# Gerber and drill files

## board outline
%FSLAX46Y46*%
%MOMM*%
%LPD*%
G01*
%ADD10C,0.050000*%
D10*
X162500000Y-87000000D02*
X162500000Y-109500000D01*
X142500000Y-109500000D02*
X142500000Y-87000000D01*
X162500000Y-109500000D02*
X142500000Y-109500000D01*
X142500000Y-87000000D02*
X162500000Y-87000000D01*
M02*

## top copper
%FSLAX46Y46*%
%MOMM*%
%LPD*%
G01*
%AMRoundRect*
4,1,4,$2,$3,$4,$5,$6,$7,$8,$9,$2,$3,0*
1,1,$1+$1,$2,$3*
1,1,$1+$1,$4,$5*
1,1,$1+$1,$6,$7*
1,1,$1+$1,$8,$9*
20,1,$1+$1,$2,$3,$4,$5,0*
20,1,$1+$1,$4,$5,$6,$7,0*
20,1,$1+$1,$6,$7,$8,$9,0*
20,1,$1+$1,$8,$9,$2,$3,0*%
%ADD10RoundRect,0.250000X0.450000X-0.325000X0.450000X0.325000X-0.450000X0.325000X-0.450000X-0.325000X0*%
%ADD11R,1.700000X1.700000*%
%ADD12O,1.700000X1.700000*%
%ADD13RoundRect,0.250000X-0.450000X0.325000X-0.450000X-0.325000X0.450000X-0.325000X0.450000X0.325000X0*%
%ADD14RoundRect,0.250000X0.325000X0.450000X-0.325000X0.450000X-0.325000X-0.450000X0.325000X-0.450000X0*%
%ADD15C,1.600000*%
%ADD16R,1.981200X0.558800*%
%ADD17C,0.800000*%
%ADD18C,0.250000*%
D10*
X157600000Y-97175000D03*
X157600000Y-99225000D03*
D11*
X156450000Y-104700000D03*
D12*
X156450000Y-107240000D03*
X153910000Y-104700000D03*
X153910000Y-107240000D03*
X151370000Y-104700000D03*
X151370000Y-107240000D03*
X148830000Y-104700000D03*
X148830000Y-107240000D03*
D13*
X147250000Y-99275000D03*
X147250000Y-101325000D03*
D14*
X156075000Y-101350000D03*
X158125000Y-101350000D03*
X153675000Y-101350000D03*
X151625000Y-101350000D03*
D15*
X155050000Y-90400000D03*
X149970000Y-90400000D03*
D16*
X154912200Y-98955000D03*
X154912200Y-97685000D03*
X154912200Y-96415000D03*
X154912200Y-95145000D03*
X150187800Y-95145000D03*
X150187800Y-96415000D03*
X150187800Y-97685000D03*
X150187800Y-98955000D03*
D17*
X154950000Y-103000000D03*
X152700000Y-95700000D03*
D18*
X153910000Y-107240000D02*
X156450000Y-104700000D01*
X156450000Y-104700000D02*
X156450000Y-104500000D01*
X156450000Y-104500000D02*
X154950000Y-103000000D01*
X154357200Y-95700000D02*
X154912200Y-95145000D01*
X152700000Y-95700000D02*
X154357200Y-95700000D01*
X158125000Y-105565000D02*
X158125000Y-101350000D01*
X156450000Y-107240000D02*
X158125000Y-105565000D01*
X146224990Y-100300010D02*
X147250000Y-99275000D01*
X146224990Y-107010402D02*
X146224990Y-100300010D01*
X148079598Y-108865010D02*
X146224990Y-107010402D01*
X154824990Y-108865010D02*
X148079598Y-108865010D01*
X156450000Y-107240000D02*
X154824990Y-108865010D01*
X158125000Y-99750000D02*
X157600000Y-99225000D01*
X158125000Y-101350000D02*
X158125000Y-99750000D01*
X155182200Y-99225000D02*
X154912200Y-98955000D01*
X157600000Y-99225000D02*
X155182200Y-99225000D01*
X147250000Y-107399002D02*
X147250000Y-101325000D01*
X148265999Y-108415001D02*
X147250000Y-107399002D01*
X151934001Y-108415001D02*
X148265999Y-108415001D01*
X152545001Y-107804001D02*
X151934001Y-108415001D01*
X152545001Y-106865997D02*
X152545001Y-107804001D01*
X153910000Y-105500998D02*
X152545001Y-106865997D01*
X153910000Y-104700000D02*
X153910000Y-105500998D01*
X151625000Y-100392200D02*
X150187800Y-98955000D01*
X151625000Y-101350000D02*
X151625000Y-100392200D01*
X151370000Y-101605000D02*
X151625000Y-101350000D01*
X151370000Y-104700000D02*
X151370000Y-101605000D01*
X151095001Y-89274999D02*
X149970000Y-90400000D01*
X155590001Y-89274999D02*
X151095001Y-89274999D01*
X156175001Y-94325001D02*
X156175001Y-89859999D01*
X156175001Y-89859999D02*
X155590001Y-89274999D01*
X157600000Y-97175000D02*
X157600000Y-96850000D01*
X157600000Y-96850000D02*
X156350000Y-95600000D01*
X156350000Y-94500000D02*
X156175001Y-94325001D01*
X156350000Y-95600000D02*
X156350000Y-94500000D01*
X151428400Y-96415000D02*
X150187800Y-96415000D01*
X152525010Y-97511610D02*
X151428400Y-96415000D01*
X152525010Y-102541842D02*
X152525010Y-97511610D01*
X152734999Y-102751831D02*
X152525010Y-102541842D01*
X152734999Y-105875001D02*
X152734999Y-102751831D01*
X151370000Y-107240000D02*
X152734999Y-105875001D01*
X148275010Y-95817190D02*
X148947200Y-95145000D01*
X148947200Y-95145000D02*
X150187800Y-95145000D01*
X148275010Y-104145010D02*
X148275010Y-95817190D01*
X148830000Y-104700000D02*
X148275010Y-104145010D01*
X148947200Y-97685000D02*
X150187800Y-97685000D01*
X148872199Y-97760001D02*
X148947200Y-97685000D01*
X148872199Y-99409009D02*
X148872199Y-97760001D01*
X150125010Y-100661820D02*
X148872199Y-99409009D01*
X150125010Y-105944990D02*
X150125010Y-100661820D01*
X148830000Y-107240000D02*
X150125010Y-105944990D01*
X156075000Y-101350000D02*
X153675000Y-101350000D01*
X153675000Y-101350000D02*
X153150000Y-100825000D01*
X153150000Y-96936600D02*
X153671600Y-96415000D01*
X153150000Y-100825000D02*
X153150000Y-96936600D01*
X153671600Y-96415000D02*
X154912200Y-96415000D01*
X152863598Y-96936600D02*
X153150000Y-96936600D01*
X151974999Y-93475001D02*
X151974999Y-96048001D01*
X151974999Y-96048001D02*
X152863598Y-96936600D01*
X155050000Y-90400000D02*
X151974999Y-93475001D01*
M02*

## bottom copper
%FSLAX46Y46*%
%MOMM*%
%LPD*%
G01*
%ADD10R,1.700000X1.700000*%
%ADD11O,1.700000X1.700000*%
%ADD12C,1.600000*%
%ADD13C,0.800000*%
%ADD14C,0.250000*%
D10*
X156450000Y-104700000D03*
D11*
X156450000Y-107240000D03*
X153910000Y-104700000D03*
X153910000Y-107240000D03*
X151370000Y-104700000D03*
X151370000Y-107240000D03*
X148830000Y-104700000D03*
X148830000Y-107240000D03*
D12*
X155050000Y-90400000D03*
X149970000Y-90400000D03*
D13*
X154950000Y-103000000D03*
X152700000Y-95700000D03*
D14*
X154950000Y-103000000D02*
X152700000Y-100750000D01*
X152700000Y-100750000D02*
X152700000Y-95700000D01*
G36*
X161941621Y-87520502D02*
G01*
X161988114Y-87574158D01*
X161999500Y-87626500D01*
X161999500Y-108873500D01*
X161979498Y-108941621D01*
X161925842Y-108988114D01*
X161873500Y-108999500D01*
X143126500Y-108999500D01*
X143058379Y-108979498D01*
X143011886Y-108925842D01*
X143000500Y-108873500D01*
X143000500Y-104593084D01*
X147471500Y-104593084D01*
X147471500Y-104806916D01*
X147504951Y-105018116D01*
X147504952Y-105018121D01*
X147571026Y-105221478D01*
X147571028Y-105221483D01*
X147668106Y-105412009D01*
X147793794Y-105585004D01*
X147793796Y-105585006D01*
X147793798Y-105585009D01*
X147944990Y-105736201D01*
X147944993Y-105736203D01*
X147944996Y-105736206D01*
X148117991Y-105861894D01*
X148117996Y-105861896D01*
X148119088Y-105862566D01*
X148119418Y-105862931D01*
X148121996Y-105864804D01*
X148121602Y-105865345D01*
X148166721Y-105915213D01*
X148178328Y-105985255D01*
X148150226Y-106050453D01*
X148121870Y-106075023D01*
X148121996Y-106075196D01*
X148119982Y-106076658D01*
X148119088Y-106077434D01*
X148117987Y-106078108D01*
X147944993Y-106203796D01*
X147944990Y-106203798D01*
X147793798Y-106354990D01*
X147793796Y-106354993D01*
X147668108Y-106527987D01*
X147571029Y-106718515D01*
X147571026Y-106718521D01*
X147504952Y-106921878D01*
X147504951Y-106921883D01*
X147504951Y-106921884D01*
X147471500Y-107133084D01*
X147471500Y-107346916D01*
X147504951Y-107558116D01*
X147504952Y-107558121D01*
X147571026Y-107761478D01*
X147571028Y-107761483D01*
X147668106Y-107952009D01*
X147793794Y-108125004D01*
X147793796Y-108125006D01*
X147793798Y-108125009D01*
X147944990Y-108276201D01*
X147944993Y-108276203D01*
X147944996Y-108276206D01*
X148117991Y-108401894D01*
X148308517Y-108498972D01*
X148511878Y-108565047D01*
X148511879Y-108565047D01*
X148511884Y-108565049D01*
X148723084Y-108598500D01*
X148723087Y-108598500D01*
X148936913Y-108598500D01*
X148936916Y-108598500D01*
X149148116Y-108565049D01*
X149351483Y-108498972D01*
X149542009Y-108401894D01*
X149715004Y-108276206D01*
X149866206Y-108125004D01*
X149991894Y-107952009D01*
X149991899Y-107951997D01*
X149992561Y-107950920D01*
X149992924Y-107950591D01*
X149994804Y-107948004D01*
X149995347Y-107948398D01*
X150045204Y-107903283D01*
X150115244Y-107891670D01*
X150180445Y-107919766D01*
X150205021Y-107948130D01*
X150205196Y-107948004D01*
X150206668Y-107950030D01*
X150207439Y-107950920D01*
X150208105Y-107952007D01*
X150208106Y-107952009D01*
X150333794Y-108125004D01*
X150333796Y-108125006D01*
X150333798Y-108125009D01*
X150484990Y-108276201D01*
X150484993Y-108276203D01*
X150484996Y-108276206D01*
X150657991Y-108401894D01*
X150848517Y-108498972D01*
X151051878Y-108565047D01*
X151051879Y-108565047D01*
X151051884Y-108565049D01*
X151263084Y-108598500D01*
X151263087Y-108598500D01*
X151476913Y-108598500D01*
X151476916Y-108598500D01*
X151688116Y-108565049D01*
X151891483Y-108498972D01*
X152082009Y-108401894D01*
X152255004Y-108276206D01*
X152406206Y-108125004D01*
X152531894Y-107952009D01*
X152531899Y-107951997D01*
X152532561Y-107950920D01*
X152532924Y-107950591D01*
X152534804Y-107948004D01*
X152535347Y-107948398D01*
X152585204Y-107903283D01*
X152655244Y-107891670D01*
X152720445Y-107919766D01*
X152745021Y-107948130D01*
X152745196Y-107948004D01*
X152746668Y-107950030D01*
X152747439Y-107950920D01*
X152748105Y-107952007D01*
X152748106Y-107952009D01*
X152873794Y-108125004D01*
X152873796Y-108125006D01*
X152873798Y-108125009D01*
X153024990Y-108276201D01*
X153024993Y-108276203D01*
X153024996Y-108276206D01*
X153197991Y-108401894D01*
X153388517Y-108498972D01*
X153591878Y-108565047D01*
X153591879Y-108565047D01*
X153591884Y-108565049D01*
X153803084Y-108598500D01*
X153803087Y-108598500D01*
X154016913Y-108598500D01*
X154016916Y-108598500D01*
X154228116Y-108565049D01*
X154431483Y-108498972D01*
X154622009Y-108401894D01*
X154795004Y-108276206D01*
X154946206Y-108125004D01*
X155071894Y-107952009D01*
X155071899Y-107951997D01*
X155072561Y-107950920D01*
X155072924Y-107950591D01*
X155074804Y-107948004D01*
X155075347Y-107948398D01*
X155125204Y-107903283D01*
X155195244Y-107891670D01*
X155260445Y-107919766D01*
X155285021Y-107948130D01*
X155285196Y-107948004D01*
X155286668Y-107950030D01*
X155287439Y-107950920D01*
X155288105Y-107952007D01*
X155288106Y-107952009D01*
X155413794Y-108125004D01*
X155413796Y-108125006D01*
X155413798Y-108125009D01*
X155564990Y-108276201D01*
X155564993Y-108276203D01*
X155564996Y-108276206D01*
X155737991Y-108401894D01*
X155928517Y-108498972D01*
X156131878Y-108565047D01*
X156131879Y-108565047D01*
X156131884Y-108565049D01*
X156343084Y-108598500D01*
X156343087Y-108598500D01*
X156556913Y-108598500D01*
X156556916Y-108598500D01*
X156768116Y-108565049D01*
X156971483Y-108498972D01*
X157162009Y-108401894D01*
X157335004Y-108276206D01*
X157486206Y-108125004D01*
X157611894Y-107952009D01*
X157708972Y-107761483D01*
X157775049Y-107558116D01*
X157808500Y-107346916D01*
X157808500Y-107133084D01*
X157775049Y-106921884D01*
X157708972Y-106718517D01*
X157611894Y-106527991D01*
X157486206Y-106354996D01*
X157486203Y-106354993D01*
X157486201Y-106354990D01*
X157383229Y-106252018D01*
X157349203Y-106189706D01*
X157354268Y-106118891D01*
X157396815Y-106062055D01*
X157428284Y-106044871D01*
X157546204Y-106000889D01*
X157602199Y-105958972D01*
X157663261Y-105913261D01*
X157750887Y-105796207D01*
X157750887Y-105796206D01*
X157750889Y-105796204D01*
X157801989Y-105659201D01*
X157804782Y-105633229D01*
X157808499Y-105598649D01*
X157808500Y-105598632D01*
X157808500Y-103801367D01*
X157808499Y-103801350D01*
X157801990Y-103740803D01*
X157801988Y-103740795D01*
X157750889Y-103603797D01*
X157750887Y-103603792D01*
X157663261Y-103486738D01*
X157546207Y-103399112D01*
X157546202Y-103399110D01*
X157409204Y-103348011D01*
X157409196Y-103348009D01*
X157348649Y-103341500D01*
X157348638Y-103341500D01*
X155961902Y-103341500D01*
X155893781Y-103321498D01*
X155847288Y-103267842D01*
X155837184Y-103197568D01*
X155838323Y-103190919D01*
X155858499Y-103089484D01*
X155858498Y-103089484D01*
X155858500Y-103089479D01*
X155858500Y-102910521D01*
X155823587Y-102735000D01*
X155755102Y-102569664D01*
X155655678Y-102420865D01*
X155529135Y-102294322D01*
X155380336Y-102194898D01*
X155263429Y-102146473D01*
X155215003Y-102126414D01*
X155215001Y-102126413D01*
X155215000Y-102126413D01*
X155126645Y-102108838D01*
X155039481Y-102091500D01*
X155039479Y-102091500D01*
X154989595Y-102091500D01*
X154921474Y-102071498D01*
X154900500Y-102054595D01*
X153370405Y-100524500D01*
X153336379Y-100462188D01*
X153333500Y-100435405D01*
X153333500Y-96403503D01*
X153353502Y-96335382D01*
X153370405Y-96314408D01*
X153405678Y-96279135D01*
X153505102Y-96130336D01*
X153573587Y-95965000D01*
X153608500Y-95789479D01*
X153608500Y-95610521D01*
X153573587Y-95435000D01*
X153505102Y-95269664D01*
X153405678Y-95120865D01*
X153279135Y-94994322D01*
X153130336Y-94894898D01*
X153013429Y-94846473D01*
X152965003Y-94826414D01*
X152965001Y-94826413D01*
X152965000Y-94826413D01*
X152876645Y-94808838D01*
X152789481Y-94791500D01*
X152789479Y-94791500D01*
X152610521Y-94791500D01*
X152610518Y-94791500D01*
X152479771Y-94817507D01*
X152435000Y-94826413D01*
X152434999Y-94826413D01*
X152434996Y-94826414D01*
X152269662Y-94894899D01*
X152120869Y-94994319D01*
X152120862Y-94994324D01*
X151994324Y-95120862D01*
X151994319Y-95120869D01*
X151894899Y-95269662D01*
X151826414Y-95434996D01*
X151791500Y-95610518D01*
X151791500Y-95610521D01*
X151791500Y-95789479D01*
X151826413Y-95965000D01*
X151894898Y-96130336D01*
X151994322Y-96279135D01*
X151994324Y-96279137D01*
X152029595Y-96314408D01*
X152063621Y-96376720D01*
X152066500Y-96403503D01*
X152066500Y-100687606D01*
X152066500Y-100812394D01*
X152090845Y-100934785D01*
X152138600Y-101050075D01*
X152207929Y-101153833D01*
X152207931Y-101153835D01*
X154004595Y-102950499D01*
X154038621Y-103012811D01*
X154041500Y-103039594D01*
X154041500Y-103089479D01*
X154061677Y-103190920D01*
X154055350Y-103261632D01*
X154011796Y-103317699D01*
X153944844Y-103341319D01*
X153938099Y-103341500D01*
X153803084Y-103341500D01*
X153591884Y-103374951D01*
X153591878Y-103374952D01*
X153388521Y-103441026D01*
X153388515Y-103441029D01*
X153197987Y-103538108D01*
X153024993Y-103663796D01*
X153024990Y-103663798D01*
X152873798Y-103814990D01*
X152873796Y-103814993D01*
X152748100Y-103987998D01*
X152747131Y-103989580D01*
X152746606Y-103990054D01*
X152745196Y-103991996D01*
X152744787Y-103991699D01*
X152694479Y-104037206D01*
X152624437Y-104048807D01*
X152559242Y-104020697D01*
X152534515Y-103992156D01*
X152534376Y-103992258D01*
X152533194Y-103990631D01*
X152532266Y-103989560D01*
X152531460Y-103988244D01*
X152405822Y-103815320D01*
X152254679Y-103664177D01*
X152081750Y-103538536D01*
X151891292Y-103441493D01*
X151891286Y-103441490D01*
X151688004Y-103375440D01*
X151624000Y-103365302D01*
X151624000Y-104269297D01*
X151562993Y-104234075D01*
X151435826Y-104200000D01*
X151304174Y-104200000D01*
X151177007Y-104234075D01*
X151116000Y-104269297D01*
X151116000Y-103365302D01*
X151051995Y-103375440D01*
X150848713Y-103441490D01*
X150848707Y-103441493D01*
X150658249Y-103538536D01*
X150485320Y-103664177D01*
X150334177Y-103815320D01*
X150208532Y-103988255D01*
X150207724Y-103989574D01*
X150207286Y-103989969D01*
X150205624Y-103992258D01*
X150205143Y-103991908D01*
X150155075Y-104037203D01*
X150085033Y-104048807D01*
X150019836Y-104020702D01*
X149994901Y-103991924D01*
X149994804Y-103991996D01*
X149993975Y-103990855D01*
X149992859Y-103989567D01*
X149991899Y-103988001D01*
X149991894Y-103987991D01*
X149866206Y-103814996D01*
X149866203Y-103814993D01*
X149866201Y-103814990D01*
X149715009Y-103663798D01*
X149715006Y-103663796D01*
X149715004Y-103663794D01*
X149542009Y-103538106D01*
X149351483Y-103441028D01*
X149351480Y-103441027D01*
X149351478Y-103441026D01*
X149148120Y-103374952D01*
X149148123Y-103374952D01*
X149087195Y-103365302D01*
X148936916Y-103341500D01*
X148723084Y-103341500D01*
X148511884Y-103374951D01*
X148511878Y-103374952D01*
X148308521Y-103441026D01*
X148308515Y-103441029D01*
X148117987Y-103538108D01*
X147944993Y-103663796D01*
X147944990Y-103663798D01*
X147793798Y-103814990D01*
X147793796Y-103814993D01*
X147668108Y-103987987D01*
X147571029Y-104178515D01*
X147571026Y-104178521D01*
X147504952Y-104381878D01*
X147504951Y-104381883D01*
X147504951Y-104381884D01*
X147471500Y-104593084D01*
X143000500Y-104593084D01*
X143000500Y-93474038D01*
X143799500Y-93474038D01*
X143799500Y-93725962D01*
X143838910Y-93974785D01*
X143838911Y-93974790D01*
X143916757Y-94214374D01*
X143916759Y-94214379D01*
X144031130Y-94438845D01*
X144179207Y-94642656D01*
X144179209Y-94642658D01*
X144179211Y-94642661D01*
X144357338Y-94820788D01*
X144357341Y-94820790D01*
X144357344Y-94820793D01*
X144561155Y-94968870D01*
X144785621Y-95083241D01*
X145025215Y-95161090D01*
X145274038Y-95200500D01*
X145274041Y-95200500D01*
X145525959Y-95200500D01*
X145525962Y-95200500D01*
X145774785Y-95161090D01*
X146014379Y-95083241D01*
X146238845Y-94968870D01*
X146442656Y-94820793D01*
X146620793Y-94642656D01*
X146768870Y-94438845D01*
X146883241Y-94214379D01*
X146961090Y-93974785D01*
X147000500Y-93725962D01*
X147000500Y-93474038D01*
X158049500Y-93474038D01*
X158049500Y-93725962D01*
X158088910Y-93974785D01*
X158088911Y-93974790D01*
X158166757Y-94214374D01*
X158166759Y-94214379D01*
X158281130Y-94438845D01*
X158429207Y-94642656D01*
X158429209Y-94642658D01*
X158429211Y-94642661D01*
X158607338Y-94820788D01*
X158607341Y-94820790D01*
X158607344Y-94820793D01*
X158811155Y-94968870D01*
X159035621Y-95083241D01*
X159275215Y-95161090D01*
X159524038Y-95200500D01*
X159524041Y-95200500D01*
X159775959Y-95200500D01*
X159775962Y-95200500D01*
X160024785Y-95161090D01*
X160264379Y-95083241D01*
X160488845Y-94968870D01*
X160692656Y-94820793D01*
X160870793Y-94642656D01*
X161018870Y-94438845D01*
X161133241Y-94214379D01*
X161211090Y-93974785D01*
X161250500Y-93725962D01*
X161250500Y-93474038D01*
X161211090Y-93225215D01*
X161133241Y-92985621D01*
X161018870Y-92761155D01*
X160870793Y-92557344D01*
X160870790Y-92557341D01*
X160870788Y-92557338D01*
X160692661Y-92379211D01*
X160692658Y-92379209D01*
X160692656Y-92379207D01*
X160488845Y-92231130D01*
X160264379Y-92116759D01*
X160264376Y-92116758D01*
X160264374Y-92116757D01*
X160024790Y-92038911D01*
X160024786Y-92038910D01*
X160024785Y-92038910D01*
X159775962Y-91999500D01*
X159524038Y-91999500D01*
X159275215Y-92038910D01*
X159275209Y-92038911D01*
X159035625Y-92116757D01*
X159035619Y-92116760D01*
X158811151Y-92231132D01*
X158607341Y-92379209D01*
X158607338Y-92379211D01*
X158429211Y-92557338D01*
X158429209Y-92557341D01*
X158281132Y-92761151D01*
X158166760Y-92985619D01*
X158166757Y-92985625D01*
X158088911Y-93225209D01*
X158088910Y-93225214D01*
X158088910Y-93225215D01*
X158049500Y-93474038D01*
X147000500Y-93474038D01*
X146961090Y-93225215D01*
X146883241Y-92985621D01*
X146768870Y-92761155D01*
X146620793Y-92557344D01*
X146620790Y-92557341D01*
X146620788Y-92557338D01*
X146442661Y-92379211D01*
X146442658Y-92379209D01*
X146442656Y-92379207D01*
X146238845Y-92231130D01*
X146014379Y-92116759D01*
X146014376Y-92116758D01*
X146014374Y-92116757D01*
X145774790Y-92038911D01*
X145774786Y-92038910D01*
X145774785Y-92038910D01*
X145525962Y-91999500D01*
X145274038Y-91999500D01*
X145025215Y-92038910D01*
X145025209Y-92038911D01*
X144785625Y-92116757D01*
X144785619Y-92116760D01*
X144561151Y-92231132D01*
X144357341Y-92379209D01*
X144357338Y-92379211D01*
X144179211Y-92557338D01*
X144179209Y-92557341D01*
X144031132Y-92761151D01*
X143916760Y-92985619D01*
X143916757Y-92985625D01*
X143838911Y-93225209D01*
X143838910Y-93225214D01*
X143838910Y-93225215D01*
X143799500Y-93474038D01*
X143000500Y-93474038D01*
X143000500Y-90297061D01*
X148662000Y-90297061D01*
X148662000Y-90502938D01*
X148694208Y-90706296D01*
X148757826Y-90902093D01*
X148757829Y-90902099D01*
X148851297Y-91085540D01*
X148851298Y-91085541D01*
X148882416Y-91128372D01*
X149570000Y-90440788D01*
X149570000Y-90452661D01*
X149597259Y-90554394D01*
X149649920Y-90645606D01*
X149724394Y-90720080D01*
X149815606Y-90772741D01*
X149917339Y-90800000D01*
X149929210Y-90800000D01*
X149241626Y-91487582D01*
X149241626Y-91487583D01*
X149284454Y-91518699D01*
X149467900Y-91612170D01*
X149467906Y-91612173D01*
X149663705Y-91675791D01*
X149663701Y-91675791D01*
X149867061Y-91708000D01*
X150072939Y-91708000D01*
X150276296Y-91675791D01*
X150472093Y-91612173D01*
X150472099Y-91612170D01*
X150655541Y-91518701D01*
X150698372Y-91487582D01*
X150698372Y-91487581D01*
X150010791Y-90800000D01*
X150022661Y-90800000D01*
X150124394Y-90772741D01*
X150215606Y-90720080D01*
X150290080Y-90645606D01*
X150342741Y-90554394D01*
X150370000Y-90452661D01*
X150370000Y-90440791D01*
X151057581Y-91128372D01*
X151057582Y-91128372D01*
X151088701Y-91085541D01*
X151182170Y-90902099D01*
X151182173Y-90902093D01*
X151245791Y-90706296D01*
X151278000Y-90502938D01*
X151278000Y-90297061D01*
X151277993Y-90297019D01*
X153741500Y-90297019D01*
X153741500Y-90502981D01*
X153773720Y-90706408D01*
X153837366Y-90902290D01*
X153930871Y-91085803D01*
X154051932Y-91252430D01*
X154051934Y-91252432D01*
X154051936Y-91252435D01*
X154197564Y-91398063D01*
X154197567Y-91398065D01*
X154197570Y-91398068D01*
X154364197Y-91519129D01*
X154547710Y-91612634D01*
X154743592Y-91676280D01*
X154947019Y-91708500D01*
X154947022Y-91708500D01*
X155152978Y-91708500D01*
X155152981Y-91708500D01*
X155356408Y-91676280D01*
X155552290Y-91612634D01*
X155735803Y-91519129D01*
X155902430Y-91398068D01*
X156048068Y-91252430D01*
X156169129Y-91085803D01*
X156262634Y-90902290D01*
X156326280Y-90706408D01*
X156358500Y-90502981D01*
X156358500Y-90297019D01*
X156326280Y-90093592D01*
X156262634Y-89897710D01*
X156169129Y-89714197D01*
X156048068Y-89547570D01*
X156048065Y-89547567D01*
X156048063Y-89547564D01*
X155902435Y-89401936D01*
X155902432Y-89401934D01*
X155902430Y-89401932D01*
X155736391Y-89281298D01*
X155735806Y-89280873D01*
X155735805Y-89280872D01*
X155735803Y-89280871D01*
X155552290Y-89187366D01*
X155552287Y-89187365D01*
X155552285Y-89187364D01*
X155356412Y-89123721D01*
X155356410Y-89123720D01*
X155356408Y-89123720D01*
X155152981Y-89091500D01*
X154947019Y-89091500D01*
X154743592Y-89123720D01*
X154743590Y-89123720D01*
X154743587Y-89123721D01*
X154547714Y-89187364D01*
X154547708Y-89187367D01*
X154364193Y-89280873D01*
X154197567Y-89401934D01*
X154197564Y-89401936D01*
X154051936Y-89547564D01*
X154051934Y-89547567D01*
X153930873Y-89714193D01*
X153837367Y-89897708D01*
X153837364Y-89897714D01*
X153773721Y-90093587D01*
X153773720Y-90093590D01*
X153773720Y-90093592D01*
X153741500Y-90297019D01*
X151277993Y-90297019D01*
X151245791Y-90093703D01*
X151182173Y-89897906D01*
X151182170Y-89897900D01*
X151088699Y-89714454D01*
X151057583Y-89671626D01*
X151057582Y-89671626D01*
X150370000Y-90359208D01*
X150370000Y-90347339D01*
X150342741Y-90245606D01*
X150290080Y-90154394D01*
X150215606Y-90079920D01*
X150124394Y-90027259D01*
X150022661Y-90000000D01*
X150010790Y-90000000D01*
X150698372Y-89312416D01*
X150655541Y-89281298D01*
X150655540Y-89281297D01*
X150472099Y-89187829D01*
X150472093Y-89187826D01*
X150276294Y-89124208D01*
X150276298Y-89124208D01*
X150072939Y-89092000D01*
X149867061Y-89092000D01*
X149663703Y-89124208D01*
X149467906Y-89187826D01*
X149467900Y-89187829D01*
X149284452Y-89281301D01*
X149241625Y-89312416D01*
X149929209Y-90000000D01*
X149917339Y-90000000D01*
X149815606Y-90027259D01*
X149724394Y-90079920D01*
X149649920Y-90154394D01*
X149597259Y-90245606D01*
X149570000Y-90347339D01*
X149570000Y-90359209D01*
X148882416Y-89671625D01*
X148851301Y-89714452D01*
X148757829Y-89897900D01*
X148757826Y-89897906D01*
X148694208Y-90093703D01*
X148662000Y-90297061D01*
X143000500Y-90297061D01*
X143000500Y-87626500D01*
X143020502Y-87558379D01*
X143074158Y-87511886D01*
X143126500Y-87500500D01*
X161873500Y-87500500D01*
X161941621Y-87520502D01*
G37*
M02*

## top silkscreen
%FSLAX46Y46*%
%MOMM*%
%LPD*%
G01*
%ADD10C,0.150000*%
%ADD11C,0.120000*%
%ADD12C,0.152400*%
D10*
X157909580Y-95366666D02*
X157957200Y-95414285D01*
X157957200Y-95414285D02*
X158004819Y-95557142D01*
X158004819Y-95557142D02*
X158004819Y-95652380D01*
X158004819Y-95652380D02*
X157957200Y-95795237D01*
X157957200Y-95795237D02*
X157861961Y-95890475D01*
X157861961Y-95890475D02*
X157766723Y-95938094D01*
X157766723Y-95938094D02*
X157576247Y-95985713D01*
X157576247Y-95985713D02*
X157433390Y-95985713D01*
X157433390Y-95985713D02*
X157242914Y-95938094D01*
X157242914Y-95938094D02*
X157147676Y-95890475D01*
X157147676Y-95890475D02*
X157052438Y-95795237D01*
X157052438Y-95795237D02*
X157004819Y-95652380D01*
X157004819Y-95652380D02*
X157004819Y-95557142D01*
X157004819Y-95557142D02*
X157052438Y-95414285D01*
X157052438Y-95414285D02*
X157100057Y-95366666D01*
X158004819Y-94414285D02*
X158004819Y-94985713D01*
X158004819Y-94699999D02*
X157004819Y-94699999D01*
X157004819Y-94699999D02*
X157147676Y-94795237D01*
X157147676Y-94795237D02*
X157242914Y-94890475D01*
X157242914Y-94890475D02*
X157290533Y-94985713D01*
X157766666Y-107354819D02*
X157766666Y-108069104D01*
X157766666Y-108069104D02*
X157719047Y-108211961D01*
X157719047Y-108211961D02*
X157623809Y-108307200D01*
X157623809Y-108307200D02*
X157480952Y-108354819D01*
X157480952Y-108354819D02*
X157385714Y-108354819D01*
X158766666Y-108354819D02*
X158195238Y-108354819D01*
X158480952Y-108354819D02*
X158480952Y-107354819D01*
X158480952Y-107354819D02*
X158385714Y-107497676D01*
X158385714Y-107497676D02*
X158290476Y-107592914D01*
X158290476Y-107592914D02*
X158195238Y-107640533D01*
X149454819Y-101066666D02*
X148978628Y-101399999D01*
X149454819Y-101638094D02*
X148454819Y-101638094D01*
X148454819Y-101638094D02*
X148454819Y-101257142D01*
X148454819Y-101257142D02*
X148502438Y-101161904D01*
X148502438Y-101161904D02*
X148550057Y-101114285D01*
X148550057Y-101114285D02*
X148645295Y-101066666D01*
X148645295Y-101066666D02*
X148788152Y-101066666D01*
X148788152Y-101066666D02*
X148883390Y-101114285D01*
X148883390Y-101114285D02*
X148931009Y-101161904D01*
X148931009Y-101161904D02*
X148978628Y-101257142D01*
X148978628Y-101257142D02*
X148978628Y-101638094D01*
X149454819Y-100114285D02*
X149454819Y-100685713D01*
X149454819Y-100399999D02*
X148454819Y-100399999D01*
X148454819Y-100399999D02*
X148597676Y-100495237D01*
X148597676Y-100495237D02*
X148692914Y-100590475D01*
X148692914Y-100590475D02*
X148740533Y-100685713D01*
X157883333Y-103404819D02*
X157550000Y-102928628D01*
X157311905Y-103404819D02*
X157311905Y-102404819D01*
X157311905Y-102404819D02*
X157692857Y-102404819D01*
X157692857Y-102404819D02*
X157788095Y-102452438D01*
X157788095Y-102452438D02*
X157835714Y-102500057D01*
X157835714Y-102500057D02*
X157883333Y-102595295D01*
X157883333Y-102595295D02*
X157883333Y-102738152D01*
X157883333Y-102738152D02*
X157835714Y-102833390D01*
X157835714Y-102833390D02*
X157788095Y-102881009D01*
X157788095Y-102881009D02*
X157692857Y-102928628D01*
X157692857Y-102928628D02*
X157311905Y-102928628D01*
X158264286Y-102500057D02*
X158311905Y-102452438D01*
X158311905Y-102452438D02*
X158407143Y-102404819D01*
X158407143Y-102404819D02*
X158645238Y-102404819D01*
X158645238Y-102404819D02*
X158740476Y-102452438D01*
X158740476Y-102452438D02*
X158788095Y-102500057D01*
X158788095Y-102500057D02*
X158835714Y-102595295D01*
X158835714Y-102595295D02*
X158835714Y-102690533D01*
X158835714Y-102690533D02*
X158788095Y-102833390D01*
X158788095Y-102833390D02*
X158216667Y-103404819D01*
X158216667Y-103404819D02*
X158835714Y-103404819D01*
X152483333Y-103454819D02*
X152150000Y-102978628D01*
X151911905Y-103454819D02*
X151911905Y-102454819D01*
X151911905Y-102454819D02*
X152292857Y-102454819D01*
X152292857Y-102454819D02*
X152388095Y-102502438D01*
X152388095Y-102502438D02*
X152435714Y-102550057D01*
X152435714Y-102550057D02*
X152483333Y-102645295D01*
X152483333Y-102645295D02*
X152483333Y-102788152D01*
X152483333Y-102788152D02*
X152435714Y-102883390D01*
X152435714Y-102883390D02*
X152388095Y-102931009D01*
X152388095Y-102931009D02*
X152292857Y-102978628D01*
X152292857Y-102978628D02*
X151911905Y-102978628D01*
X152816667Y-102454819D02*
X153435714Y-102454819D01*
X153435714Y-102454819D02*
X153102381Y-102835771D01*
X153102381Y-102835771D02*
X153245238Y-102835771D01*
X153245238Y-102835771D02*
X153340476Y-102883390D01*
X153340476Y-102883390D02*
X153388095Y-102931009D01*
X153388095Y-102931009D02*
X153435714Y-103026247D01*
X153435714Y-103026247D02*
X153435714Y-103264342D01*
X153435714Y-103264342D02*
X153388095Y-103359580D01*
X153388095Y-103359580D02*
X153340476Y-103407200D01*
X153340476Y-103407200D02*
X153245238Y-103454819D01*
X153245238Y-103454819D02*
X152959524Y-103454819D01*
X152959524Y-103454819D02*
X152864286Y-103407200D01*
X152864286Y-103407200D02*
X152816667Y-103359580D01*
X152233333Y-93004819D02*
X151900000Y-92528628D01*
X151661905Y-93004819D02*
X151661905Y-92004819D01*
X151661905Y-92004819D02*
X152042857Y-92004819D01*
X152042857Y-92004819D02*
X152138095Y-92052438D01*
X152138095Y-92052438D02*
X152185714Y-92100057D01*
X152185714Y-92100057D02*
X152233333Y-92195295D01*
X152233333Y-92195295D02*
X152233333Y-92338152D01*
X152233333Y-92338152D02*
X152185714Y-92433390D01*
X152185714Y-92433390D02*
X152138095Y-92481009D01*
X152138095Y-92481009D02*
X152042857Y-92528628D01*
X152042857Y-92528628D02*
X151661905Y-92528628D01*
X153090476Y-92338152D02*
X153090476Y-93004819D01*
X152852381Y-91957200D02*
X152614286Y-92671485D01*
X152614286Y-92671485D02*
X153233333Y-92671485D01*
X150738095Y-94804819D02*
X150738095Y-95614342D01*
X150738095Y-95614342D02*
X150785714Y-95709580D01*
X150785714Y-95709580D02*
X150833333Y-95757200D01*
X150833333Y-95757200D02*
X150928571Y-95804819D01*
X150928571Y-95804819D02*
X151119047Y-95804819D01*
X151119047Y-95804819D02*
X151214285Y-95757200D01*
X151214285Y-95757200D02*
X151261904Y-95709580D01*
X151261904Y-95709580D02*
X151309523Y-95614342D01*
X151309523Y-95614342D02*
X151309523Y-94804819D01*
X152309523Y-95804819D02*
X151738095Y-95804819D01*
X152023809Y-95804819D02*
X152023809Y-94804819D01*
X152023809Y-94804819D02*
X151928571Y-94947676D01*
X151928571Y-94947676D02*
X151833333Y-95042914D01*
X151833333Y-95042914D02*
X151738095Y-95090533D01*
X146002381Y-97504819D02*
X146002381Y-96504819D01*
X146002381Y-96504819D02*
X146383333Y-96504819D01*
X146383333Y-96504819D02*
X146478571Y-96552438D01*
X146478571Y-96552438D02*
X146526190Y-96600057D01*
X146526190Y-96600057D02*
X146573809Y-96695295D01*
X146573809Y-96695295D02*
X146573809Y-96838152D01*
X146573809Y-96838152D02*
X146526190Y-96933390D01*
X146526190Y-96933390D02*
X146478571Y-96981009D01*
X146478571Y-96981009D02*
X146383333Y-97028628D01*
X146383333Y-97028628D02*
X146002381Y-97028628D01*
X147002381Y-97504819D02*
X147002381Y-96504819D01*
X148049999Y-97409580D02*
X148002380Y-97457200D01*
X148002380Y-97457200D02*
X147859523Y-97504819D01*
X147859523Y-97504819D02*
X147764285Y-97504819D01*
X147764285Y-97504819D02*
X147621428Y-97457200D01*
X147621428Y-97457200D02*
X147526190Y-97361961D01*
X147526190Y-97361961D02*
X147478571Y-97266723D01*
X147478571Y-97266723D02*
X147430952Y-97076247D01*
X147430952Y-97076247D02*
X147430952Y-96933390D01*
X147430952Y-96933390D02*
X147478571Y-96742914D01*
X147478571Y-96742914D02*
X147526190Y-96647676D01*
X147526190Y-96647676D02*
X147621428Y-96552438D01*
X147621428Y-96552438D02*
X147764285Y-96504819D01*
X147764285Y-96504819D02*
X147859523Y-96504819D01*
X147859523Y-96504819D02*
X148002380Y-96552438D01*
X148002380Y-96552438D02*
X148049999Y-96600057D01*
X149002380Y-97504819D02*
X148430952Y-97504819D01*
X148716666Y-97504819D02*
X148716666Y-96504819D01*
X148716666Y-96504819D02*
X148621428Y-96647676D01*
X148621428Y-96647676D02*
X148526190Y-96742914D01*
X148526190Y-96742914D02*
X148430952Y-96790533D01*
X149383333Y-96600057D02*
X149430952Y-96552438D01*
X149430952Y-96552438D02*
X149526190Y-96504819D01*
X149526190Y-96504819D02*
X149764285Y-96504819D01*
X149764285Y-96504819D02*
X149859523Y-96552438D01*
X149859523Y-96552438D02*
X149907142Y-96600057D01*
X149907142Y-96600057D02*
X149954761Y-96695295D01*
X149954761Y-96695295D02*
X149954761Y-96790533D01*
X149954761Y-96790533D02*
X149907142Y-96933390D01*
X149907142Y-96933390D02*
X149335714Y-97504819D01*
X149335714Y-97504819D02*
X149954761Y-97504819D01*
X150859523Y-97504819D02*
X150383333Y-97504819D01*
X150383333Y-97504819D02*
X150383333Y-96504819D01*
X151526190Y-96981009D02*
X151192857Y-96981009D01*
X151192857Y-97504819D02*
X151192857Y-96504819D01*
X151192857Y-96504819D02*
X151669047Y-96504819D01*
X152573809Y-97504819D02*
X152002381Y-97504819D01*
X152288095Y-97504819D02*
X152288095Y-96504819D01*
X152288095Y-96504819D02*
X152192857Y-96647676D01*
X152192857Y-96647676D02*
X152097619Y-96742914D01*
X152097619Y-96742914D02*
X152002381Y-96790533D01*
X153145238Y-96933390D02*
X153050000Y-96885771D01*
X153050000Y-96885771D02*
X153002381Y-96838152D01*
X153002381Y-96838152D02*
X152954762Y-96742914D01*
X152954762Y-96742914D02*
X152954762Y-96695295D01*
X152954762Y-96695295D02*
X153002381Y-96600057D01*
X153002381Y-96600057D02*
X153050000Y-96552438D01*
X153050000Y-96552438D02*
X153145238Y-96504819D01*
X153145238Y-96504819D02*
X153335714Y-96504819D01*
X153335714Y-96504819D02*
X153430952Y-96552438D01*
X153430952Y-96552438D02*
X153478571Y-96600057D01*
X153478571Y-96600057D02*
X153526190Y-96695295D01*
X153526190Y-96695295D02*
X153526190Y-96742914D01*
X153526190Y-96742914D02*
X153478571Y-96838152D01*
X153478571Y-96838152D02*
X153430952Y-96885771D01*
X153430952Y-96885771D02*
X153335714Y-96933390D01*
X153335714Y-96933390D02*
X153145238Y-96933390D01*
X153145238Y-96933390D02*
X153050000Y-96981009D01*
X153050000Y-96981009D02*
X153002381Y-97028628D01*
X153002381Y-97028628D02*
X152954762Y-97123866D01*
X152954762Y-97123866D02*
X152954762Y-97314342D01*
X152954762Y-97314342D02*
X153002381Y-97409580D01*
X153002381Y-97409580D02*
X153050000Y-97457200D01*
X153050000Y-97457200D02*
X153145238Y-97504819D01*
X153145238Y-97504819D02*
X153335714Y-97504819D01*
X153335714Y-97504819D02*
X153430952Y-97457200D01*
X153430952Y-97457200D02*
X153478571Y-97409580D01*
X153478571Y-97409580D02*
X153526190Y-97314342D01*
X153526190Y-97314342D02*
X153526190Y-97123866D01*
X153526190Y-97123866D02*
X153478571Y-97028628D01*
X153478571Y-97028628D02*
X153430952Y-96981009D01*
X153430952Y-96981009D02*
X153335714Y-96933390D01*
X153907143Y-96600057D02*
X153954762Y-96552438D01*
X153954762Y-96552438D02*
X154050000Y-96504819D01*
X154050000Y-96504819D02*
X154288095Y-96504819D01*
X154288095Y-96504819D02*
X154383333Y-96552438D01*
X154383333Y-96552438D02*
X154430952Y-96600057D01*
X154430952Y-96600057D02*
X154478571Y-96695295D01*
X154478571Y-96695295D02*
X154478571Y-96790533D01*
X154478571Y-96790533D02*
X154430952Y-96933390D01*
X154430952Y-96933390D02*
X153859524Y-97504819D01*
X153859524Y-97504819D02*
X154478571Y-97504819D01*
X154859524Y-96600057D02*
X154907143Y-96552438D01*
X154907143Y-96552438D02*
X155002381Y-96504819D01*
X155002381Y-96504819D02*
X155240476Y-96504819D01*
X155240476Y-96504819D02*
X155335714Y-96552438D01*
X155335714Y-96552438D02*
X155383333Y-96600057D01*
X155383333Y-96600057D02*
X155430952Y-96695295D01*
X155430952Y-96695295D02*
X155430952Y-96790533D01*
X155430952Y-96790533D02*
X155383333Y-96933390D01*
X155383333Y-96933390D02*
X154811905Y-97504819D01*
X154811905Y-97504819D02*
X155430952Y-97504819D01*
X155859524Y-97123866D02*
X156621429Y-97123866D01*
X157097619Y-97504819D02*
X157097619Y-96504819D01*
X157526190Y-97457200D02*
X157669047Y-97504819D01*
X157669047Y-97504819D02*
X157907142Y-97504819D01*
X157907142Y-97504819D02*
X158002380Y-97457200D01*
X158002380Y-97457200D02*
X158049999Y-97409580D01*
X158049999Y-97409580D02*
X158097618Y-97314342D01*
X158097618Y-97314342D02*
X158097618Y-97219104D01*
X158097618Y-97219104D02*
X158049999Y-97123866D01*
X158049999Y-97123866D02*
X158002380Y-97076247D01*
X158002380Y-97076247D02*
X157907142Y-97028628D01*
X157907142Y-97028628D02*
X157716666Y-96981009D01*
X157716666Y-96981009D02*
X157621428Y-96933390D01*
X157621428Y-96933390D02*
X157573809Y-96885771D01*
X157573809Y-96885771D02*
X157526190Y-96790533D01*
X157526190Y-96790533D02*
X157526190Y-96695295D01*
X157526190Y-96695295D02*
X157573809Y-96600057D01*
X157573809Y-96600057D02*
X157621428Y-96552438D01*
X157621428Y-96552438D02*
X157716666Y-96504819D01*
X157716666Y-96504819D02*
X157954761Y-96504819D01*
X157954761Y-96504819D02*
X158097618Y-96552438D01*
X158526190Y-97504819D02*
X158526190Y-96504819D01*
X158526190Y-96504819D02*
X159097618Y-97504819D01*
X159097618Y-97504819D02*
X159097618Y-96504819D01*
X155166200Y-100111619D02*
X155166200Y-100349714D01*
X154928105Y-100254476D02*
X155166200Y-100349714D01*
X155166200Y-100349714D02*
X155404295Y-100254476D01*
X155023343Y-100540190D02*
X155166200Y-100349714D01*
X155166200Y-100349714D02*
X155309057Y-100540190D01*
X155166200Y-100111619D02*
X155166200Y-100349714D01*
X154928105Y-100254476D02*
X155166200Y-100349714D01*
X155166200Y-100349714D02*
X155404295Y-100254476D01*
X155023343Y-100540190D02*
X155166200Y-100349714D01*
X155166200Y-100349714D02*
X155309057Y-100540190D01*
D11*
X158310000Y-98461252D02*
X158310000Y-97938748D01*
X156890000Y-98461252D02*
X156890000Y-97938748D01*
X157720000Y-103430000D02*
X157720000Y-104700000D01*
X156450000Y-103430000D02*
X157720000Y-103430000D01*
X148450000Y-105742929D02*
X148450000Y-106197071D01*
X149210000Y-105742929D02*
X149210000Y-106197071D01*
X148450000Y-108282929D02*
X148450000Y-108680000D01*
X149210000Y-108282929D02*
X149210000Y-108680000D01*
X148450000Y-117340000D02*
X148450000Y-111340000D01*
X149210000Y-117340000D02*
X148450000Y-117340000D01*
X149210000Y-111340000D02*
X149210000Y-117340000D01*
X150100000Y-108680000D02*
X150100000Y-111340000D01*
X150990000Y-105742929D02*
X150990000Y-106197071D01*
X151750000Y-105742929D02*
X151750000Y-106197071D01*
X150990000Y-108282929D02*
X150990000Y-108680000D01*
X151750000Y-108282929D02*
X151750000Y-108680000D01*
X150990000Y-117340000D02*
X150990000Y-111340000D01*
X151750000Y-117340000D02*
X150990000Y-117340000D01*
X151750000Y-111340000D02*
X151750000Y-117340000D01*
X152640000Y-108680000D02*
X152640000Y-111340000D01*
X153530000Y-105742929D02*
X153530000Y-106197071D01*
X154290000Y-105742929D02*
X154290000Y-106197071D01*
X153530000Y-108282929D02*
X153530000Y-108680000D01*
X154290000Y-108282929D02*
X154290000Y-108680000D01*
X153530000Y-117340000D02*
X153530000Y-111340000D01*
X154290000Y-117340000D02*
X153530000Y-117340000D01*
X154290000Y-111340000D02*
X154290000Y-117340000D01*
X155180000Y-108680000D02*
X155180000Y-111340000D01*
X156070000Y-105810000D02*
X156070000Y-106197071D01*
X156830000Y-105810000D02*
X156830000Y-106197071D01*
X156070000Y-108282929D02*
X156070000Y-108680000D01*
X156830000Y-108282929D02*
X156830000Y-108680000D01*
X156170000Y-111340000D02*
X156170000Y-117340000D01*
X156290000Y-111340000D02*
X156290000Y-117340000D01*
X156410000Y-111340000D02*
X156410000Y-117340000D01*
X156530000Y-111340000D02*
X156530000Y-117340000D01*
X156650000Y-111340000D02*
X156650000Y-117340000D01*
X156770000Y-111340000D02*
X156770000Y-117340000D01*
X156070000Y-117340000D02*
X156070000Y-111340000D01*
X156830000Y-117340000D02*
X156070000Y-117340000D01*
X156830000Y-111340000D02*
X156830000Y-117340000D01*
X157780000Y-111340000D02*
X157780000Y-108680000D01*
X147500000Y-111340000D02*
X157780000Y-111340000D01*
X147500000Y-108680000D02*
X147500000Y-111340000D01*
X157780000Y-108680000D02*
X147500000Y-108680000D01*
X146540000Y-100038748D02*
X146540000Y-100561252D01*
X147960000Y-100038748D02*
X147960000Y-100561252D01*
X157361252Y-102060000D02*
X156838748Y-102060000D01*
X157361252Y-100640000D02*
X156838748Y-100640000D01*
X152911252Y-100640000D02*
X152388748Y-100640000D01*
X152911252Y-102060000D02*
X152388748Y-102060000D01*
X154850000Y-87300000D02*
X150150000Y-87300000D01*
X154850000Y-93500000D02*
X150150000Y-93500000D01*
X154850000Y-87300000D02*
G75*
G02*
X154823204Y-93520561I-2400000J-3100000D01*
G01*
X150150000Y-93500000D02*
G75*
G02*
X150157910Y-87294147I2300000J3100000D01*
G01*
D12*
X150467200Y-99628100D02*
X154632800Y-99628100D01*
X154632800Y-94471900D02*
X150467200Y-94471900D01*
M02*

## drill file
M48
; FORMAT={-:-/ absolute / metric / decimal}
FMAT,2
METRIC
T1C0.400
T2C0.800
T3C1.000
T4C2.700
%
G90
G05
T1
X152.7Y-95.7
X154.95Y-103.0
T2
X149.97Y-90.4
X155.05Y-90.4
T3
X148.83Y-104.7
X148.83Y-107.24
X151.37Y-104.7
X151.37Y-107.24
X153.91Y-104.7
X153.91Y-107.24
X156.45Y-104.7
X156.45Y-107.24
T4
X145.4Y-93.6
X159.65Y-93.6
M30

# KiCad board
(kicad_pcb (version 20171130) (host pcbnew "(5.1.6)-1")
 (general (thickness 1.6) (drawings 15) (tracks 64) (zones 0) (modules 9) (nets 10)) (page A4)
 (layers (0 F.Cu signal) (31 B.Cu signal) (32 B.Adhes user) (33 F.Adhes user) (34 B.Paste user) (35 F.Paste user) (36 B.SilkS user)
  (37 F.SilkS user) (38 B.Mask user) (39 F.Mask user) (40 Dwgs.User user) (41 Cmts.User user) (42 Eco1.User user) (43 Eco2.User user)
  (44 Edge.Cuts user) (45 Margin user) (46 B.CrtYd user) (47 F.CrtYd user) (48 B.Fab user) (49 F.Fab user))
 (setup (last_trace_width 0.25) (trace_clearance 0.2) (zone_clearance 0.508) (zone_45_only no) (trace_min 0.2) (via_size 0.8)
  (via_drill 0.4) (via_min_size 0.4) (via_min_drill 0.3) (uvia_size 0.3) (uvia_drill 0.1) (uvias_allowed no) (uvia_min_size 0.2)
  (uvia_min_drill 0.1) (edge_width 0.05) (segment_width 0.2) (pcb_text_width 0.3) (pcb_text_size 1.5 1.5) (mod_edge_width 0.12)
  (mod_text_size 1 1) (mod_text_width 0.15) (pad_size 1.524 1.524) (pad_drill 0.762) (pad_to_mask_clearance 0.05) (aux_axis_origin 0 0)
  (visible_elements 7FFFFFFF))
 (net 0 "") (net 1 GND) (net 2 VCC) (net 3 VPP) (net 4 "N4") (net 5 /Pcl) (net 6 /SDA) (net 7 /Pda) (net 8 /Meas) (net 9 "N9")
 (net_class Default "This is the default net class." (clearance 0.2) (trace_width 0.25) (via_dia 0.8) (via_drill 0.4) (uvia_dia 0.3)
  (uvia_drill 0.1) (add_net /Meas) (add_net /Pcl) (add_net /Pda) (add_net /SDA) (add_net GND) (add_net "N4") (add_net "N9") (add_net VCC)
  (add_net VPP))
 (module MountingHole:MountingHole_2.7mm (layer F.Cu) (at 145.4 93.6)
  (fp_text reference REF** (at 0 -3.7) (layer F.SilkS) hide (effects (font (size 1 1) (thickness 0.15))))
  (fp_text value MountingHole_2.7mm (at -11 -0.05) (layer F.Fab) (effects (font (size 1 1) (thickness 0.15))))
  (pad 1 np_thru_hole circle (at 0 0) (size 2.7 2.7) (drill 2.7) (layers *.Cu *.Mask)))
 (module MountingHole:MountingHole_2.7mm (layer F.Cu) (at 159.65 93.6)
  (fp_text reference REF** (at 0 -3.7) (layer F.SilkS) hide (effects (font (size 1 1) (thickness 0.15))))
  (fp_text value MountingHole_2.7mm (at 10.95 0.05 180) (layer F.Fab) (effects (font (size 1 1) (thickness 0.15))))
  (pad 1 np_thru_hole circle (at 0 0) (size 2.7 2.7) (drill 2.7) (layers *.Cu *.Mask)))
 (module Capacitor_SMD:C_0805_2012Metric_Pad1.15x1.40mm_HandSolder (layer F.Cu) (at 157.6 98.2 90)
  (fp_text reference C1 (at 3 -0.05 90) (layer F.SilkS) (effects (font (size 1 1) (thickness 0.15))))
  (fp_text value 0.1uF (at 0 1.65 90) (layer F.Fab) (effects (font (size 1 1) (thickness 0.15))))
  (fp_line (start -0.261252 0.71) (end 0.261252 0.71) (layer F.SilkS) (width 0.12))
  (fp_line (start -0.261252 -0.71) (end 0.261252 -0.71) (layer F.SilkS) (width 0.12))
  (pad 2 smd roundrect (at 1.025 0 90) (size 1.15 1.4) (layers F.Cu F.Paste F.Mask) (roundrect_rratio 0.217391) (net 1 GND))
  (pad 1 smd roundrect (at -1.025 0 90) (size 1.15 1.4) (layers F.Cu F.Paste F.Mask) (roundrect_rratio 0.217391) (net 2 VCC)))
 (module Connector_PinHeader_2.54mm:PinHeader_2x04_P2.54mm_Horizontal (layer F.Cu) (at 156.45 104.7 270)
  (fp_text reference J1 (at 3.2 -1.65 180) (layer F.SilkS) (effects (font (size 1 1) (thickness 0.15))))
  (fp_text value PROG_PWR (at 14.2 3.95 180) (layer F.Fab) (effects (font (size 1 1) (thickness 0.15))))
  (fp_line (start -1.27 -1.27) (end 0 -1.27) (layer F.SilkS) (width 0.12))
  (fp_line (start -1.27 0) (end -1.27 -1.27) (layer F.SilkS) (width 0.12))
  (fp_line (start 1.042929 8) (end 1.497071 8) (layer F.SilkS) (width 0.12))
  (fp_line (start 1.042929 7.24) (end 1.497071 7.24) (layer F.SilkS) (width 0.12))
  (fp_line (start 3.582929 8) (end 3.98 8) (layer F.SilkS) (width 0.12))
  (fp_line (start 3.582929 7.24) (end 3.98 7.24) (layer F.SilkS) (width 0.12))
  (fp_line (start 12.64 8) (end 6.64 8) (layer F.SilkS) (width 0.12))
  (fp_line (start 12.64 7.24) (end 12.64 8) (layer F.SilkS) (width 0.12))
  (fp_line (start 6.64 7.24) (end 12.64 7.24) (layer F.SilkS) (width 0.12))
  (fp_line (start 3.98 6.35) (end 6.64 6.35) (layer F.SilkS) (width 0.12))
  (fp_line (start 1.042929 5.46) (end 1.497071 5.46) (layer F.SilkS) (width 0.12))
  (fp_line (start 1.042929 4.7) (end 1.497071 4.7) (layer F.SilkS) (width 0.12))
  (fp_line (start 3.582929 5.46) (end 3.98 5.46) (layer F.SilkS) (width 0.12))
  (fp_line (start 3.582929 4.7) (end 3.98 4.7) (layer F.SilkS) (width 0.12))
  (fp_line (start 12.64 5.46) (end 6.64 5.46) (layer F.SilkS) (width 0.12))
  (fp_line (start 12.64 4.7) (end 12.64 5.46) (layer F.SilkS) (width 0.12))
  (fp_line (start 6.64 4.7) (end 12.64 4.7) (layer F.SilkS) (width 0.12))
  (fp_line (start 3.98 3.81) (end 6.64 3.81) (layer F.SilkS) (width 0.12))
  (fp_line (start 1.042929 2.92) (end 1.497071 2.92) (layer F.SilkS) (width 0.12))
  (fp_line (start 1.042929 2.16) (end 1.497071 2.16) (layer F.SilkS) (width 0.12))
  (fp_line (start 3.582929 2.92) (end 3.98 2.92) (layer F.SilkS) (width 0.12))
  (fp_line (start 3.582929 2.16) (end 3.98 2.16) (layer F.SilkS) (width 0.12))
  (fp_line (start 12.64 2.92) (end 6.64 2.92) (layer F.SilkS) (width 0.12))
  (fp_line (start 12.64 2.16) (end 12.64 2.92) (layer F.SilkS) (width 0.12))
  (fp_line (start 6.64 2.16) (end 12.64 2.16) (layer F.SilkS) (width 0.12))
  (fp_line (start 3.98 1.27) (end 6.64 1.27) (layer F.SilkS) (width 0.12))
  (fp_line (start 1.11 0.38) (end 1.497071 0.38) (layer F.SilkS) (width 0.12))
  (fp_line (start 1.11 -0.38) (end 1.497071 -0.38) (layer F.SilkS) (width 0.12))
  (fp_line (start 3.582929 0.38) (end 3.98 0.38) (layer F.SilkS) (width 0.12))
  (fp_line (start 3.582929 -0.38) (end 3.98 -0.38) (layer F.SilkS) (width 0.12))
  (fp_line (start 6.64 0.28) (end 12.64 0.28) (layer F.SilkS) (width 0.12))
  (fp_line (start 6.64 0.16) (end 12.64 0.16) (layer F.SilkS) (width 0.12))
  (fp_line (start 6.64 0.04) (end 12.64 0.04) (layer F.SilkS) (width 0.12))
  (fp_line (start 6.64 -0.08) (end 12.64 -0.08) (layer F.SilkS) (width 0.12))
  (fp_line (start 6.64 -0.2) (end 12.64 -0.2) (layer F.SilkS) (width 0.12))
  (fp_line (start 6.64 -0.32) (end 12.64 -0.32) (layer F.SilkS) (width 0.12))
  (fp_line (start 12.64 0.38) (end 6.64 0.38) (layer F.SilkS) (width 0.12))
  (fp_line (start 12.64 -0.38) (end 12.64 0.38) (layer F.SilkS) (width 0.12))
  (fp_line (start 6.64 -0.38) (end 12.64 -0.38) (layer F.SilkS) (width 0.12))
  (fp_line (start 6.64 -1.33) (end 3.98 -1.33) (layer F.SilkS) (width 0.12))
  (fp_line (start 6.64 8.95) (end 6.64 -1.33) (layer F.SilkS) (width 0.12))
  (fp_line (start 3.98 8.95) (end 6.64 8.95) (layer F.SilkS) (width 0.12))
  (fp_line (start 3.98 -1.33) (end 3.98 8.95) (layer F.SilkS) (width 0.12))
  (pad 1 thru_hole rect (at 0 0 270) (size 1.7 1.7) (drill 1) (layers *.Cu *.Mask) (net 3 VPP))
  (pad 2 thru_hole oval (at 2.54 0 270) (size 1.7 1.7) (drill 1) (layers *.Cu *.Mask) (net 2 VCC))
  (pad 3 thru_hole oval (at 0 2.54 270) (size 1.7 1.7) (drill 1) (layers *.Cu *.Mask) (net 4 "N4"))
  (pad 4 thru_hole oval (at 2.54 2.54 270) (size 1.7 1.7) (drill 1) (layers *.Cu *.Mask) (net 3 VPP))
  (pad 5 thru_hole oval (at 0 5.08 270) (size 1.7 1.7) (drill 1) (layers *.Cu *.Mask) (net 1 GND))
  (pad 6 thru_hole oval (at 2.54 5.08 270) (size 1.7 1.7) (drill 1) (layers *.Cu *.Mask) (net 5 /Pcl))
  (pad 7 thru_hole oval (at 0 7.62 270) (size 1.7 1.7) (drill 1) (layers *.Cu *.Mask) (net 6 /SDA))
  (pad 8 thru_hole oval (at 2.54 7.62 270) (size 1.7 1.7) (drill 1) (layers *.Cu *.Mask) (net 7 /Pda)))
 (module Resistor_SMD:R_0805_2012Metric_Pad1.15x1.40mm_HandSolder (layer F.Cu) (at 147.25 100.3 270)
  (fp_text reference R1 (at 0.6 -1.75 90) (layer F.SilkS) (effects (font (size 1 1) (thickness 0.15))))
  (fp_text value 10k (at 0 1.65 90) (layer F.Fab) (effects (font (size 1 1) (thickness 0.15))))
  (fp_line (start -0.261252 0.71) (end 0.261252 0.71) (layer F.SilkS) (width 0.12))
  (fp_line (start -0.261252 -0.71) (end 0.261252 -0.71) (layer F.SilkS) (width 0.12))
  (pad 1 smd roundrect (at -1.025 0 270) (size 1.15 1.4) (layers F.Cu F.Paste F.Mask) (roundrect_rratio 0.217391) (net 2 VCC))
  (pad 2 smd roundrect (at 1.025 0 270) (size 1.15 1.4) (layers F.Cu F.Paste F.Mask) (roundrect_rratio 0.217391) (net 4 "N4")))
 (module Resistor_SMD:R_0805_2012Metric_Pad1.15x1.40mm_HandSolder (layer F.Cu) (at 157.1 101.35 180)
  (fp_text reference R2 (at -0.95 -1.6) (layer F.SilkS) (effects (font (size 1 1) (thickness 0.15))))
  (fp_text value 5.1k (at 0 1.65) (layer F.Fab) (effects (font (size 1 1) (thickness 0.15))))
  (fp_line (start -0.261252 -0.71) (end 0.261252 -0.71) (layer F.SilkS) (width 0.12))
  (fp_line (start -0.261252 0.71) (end 0.261252 0.71) (layer F.SilkS) (width 0.12))
  (pad 2 smd roundrect (at 1.025 0 180) (size 1.15 1.4) (layers F.Cu F.Paste F.Mask) (roundrect_rratio 0.217391) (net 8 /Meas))
  (pad 1 smd roundrect (at -1.025 0 180) (size 1.15 1.4) (layers F.Cu F.Paste F.Mask) (roundrect_rratio 0.217391) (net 2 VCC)))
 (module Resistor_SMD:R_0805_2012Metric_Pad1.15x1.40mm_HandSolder (layer F.Cu) (at 152.65 101.35 180)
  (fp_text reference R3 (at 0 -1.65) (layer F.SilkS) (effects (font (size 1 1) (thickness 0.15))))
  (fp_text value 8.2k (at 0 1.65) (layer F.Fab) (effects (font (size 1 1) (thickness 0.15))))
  (fp_line (start -0.261252 0.71) (end 0.261252 0.71) (layer F.SilkS) (width 0.12))
  (fp_line (start -0.261252 -0.71) (end 0.261252 -0.71) (layer F.SilkS) (width 0.12))
  (pad 1 smd roundrect (at -1.025 0 180) (size 1.15 1.4) (layers F.Cu F.Paste F.Mask) (roundrect_rratio 0.217391) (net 8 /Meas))
  (pad 2 smd roundrect (at 1.025 0 180) (size 1.15 1.4) (layers F.Cu F.Paste F.Mask) (roundrect_rratio 0.217391) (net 1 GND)))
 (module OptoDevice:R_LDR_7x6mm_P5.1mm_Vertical (layer F.Cu) (at 155.05 90.4 180)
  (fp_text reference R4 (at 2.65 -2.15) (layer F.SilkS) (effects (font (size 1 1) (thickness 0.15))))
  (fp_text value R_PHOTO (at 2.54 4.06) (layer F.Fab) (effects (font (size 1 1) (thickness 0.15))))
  (fp_line (start 0.2 3.1) (end 4.9 3.1) (layer F.SilkS) (width 0.12))
  (fp_line (start 0.2 -3.1) (end 4.9 -3.1) (layer F.SilkS) (width 0.12))
  (fp_arc (start 2.6 0) (end 0.2 3.1) (angle 105) (layer F.SilkS) (width 0.12))
  (fp_arc (start 2.6 0) (end 4.9 -3.1) (angle 107) (layer F.SilkS) (width 0.12))
  (pad 1 thru_hole circle (at 0 0 180) (size 1.6 1.6) (drill 0.8) (layers *.Cu *.Mask) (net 8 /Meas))
  (pad 2 thru_hole circle (at 5.08 0 180) (size 1.6 1.6) (drill 0.8) (layers *.Cu *.Mask) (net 1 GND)))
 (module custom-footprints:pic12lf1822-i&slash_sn (layer F.Cu) (at 152.55 97.05 180)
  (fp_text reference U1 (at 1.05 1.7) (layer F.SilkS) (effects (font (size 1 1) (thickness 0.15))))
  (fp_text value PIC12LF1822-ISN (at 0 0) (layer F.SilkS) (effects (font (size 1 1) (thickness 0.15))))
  (fp_line (start 2.0828 -2.5781) (end -2.0828 -2.5781) (layer F.SilkS) (width 0.1524))
  (fp_line (start -2.0828 2.5781) (end 2.0828 2.5781) (layer F.SilkS) (width 0.1524))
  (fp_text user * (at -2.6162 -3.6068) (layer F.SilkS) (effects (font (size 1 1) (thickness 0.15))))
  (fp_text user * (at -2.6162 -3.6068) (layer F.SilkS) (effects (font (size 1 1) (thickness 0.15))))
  (pad 1 smd rect (at -2.3622 -1.905 180) (size 1.9812 0.5588) (layers F.Cu F.Paste F.Mask) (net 2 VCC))
  (pad 2 smd rect (at -2.3622 -0.635 180) (size 1.9812 0.5588) (layers F.Cu F.Paste F.Mask) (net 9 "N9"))
  (pad 3 smd rect (at -2.3622 0.635 180) (size 1.9812 0.5588) (layers F.Cu F.Paste F.Mask) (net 8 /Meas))
  (pad 4 smd rect (at -2.3622 1.905 180) (size 1.9812 0.5588) (layers F.Cu F.Paste F.Mask) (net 3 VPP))
  (pad 5 smd rect (at 2.3622 1.905 180) (size 1.9812 0.5588) (layers F.Cu F.Paste F.Mask) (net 6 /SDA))
  (pad 6 smd rect (at 2.3622 0.635 180) (size 1.9812 0.5588) (layers F.Cu F.Paste F.Mask) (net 5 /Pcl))
  (pad 7 smd rect (at 2.3622 -0.635 180) (size 1.9812 0.5588) (layers F.Cu F.Paste F.Mask) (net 7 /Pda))
  (pad 8 smd rect (at 2.3622 -1.905 180) (size 1.9812 0.5588) (layers F.Cu F.Paste F.Mask) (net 1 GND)))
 (gr_line (start 162.5 87) (end 162.5 109.5) (layer Edge.Cuts) (width 0.05))
 (gr_line (start 142.5 109.5) (end 142.5 87) (layer Edge.Cuts) (width 0.05))
 (gr_line (start 162.5 109.5) (end 142.5 109.5) (layer Edge.Cuts) (width 0.05))
 (gr_line (start 142.5 87) (end 162.5 87) (layer Edge.Cuts) (width 0.05))
 (segment (start 153.91 107.24) (end 156.45 104.7) (width 0.25) (layer F.Cu) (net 3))
 (via (at 154.95 103) (size 0.8) (drill 0.4) (layers F.Cu B.Cu) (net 3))
 (segment (start 156.45 104.7) (end 156.45 104.5) (width 0.25) (layer F.Cu) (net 3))
 (segment (start 156.45 104.5) (end 154.95 103) (width 0.25) (layer F.Cu) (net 3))
 (segment (start 154.95 103) (end 152.7 100.75) (width 0.25) (layer B.Cu) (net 3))
 (via (at 152.7 95.7) (size 0.8) (drill 0.4) (layers F.Cu B.Cu) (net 3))
 (segment (start 152.7 100.75) (end 152.7 95.7) (width 0.25) (layer B.Cu) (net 3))
 (segment (start 154.3572 95.7) (end 154.9122 95.145) (width 0.25) (layer F.Cu) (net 3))
 (segment (start 152.7 95.7) (end 154.3572 95.7) (width 0.25) (layer F.Cu) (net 3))
 (segment (start 158.125 105.565) (end 158.125 101.35) (width 0.25) (layer F.Cu) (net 2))
 (segment (start 156.45 107.24) (end 158.125 105.565) (width 0.25) (layer F.Cu) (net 2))
 (segment (start 146.22499 100.30001) (end 147.25 99.275) (width 0.25) (layer F.Cu) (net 2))
 (segment (start 146.22499 107.010402) (end 146.22499 100.30001) (width 0.25) (layer F.Cu) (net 2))
 (segment (start 148.079598 108.86501) (end 146.22499 107.010402) (width 0.25) (layer F.Cu) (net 2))
 (segment (start 154.82499 108.86501) (end 148.079598 108.86501) (width 0.25) (layer F.Cu) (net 2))
 (segment (start 156.45 107.24) (end 154.82499 108.86501) (width 0.25) (layer F.Cu) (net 2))
 (segment (start 158.125 99.75) (end 157.6 99.225) (width 0.25) (layer F.Cu) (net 2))
 (segment (start 158.125 101.35) (end 158.125 99.75) (width 0.25) (layer F.Cu) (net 2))
 (segment (start 155.1822 99.225) (end 154.9122 98.955) (width 0.25) (layer F.Cu) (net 2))
 (segment (start 157.6 99.225) (end 155.1822 99.225) (width 0.25) (layer F.Cu) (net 2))
 (segment (start 147.25 107.399002) (end 147.25 101.325) (width 0.25) (layer F.Cu) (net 4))
 (segment (start 148.265999 108.415001) (end 147.25 107.399002) (width 0.25) (layer F.Cu) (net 4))
 (segment (start 151.934001 108.415001) (end 148.265999 108.415001) (width 0.25) (layer F.Cu) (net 4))
 (segment (start 152.545001 107.804001) (end 151.934001 108.415001) (width 0.25) (layer F.Cu) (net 4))
 (segment (start 152.545001 106.865997) (end 152.545001 107.804001) (width 0.25) (layer F.Cu) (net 4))
 (segment (start 153.91 105.500998) (end 152.545001 106.865997) (width 0.25) (layer F.Cu) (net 4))
 (segment (start 153.91 104.7) (end 153.91 105.500998) (width 0.25) (layer F.Cu) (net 4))
 (segment (start 151.625 100.3922) (end 150.1878 98.955) (width 0.25) (layer F.Cu) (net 1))
 (segment (start 151.625 101.35) (end 151.625 100.3922) (width 0.25) (layer F.Cu) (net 1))
 (segment (start 151.37 101.605) (end 151.625 101.35) (width 0.25) (layer F.Cu) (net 1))
 (segment (start 151.37 104.7) (end 151.37 101.605) (width 0.25) (layer F.Cu) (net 1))
 (segment (start 151.095001 89.274999) (end 149.97 90.4) (width 0.25) (layer F.Cu) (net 1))
 (segment (start 155.590001 89.274999) (end 151.095001 89.274999) (width 0.25) (layer F.Cu) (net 1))
 (segment (start 156.175001 94.325001) (end 156.175001 89.859999) (width 0.25) (layer F.Cu) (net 1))
 (segment (start 156.175001 89.859999) (end 155.590001 89.274999) (width 0.25) (layer F.Cu) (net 1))
 (segment (start 157.6 97.175) (end 157.6 96.85) (width 0.25) (layer F.Cu) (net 1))
 (segment (start 157.6 96.85) (end 156.35 95.6) (width 0.25) (layer F.Cu) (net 1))
 (segment (start 156.35 94.5) (end 156.175001 94.325001) (width 0.25) (layer F.Cu) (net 1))
 (segment (start 156.35 95.6) (end 156.35 94.5) (width 0.25) (layer F.Cu) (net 1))
 (segment (start 151.4284 96.415) (end 150.1878 96.415) (width 0.25) (layer F.Cu) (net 5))
 (segment (start 152.52501 97.51161) (end 151.4284 96.415) (width 0.25) (layer F.Cu) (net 5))
 (segment (start 152.52501 102.541842) (end 152.52501 97.51161) (width 0.25) (layer F.Cu) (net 5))
 (segment (start 152.734999 102.751831) (end 152.52501 102.541842) (width 0.25) (layer F.Cu) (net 5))
 (segment (start 152.734999 105.875001) (end 152.734999 102.751831) (width 0.25) (layer F.Cu) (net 5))
 (segment (start 151.37 107.24) (end 152.734999 105.875001) (width 0.25) (layer F.Cu) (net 5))
 (segment (start 148.27501 95.81719) (end 148.9472 95.145) (width 0.25) (layer F.Cu) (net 6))
 (segment (start 148.9472 95.145) (end 150.1878 95.145) (width 0.25) (layer F.Cu) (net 6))
 (segment (start 148.27501 104.14501) (end 148.27501 95.81719) (width 0.25) (layer F.Cu) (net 6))
 (segment (start 148.83 104.7) (end 148.27501 104.14501) (width 0.25) (layer F.Cu) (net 6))
 (segment (start 148.9472 97.685) (end 150.1878 97.685) (width 0.25) (layer F.Cu) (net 7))
 (segment (start 148.872199 97.760001) (end 148.9472 97.685) (width 0.25) (layer F.Cu) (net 7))
 (segment (start 148.872199 99.409009) (end 148.872199 97.760001) (width 0.25) (layer F.Cu) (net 7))
 (segment (start 150.12501 100.66182) (end 148.872199 99.409009) (width 0.25) (layer F.Cu) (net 7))
 (segment (start 150.12501 105.94499) (end 150.12501 100.66182) (width 0.25) (layer F.Cu) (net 7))
 (segment (start 148.83 107.24) (end 150.12501 105.94499) (width 0.25) (layer F.Cu) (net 7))
 (segment (start 156.075 101.35) (end 153.675 101.35) (width 0.25) (layer F.Cu) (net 8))
 (segment (start 153.675 101.35) (end 153.15 100.825) (width 0.25) (layer F.Cu) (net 8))
 (segment (start 153.15 96.9366) (end 153.6716 96.415) (width 0.25) (layer F.Cu) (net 8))
 (segment (start 153.15 100.825) (end 153.15 96.9366) (width 0.25) (layer F.Cu) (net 8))
 (segment (start 153.6716 96.415) (end 154.9122 96.415) (width 0.25) (layer F.Cu) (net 8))
 (segment (start 152.863598 96.9366) (end 153.15 96.9366) (width 0.25) (layer F.Cu) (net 8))
 (segment (start 151.974999 93.475001) (end 151.974999 96.048001) (width 0.25) (layer F.Cu) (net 8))
 (segment (start 151.974999 96.048001) (end 152.863598 96.9366) (width 0.25) (layer F.Cu) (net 8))
 (segment (start 155.05 90.4) (end 151.974999 93.475001) (width 0.25) (layer F.Cu) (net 8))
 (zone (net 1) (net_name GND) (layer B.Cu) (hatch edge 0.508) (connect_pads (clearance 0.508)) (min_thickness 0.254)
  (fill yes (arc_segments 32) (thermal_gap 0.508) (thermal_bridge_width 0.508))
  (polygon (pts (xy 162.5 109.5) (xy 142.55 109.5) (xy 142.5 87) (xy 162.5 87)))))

